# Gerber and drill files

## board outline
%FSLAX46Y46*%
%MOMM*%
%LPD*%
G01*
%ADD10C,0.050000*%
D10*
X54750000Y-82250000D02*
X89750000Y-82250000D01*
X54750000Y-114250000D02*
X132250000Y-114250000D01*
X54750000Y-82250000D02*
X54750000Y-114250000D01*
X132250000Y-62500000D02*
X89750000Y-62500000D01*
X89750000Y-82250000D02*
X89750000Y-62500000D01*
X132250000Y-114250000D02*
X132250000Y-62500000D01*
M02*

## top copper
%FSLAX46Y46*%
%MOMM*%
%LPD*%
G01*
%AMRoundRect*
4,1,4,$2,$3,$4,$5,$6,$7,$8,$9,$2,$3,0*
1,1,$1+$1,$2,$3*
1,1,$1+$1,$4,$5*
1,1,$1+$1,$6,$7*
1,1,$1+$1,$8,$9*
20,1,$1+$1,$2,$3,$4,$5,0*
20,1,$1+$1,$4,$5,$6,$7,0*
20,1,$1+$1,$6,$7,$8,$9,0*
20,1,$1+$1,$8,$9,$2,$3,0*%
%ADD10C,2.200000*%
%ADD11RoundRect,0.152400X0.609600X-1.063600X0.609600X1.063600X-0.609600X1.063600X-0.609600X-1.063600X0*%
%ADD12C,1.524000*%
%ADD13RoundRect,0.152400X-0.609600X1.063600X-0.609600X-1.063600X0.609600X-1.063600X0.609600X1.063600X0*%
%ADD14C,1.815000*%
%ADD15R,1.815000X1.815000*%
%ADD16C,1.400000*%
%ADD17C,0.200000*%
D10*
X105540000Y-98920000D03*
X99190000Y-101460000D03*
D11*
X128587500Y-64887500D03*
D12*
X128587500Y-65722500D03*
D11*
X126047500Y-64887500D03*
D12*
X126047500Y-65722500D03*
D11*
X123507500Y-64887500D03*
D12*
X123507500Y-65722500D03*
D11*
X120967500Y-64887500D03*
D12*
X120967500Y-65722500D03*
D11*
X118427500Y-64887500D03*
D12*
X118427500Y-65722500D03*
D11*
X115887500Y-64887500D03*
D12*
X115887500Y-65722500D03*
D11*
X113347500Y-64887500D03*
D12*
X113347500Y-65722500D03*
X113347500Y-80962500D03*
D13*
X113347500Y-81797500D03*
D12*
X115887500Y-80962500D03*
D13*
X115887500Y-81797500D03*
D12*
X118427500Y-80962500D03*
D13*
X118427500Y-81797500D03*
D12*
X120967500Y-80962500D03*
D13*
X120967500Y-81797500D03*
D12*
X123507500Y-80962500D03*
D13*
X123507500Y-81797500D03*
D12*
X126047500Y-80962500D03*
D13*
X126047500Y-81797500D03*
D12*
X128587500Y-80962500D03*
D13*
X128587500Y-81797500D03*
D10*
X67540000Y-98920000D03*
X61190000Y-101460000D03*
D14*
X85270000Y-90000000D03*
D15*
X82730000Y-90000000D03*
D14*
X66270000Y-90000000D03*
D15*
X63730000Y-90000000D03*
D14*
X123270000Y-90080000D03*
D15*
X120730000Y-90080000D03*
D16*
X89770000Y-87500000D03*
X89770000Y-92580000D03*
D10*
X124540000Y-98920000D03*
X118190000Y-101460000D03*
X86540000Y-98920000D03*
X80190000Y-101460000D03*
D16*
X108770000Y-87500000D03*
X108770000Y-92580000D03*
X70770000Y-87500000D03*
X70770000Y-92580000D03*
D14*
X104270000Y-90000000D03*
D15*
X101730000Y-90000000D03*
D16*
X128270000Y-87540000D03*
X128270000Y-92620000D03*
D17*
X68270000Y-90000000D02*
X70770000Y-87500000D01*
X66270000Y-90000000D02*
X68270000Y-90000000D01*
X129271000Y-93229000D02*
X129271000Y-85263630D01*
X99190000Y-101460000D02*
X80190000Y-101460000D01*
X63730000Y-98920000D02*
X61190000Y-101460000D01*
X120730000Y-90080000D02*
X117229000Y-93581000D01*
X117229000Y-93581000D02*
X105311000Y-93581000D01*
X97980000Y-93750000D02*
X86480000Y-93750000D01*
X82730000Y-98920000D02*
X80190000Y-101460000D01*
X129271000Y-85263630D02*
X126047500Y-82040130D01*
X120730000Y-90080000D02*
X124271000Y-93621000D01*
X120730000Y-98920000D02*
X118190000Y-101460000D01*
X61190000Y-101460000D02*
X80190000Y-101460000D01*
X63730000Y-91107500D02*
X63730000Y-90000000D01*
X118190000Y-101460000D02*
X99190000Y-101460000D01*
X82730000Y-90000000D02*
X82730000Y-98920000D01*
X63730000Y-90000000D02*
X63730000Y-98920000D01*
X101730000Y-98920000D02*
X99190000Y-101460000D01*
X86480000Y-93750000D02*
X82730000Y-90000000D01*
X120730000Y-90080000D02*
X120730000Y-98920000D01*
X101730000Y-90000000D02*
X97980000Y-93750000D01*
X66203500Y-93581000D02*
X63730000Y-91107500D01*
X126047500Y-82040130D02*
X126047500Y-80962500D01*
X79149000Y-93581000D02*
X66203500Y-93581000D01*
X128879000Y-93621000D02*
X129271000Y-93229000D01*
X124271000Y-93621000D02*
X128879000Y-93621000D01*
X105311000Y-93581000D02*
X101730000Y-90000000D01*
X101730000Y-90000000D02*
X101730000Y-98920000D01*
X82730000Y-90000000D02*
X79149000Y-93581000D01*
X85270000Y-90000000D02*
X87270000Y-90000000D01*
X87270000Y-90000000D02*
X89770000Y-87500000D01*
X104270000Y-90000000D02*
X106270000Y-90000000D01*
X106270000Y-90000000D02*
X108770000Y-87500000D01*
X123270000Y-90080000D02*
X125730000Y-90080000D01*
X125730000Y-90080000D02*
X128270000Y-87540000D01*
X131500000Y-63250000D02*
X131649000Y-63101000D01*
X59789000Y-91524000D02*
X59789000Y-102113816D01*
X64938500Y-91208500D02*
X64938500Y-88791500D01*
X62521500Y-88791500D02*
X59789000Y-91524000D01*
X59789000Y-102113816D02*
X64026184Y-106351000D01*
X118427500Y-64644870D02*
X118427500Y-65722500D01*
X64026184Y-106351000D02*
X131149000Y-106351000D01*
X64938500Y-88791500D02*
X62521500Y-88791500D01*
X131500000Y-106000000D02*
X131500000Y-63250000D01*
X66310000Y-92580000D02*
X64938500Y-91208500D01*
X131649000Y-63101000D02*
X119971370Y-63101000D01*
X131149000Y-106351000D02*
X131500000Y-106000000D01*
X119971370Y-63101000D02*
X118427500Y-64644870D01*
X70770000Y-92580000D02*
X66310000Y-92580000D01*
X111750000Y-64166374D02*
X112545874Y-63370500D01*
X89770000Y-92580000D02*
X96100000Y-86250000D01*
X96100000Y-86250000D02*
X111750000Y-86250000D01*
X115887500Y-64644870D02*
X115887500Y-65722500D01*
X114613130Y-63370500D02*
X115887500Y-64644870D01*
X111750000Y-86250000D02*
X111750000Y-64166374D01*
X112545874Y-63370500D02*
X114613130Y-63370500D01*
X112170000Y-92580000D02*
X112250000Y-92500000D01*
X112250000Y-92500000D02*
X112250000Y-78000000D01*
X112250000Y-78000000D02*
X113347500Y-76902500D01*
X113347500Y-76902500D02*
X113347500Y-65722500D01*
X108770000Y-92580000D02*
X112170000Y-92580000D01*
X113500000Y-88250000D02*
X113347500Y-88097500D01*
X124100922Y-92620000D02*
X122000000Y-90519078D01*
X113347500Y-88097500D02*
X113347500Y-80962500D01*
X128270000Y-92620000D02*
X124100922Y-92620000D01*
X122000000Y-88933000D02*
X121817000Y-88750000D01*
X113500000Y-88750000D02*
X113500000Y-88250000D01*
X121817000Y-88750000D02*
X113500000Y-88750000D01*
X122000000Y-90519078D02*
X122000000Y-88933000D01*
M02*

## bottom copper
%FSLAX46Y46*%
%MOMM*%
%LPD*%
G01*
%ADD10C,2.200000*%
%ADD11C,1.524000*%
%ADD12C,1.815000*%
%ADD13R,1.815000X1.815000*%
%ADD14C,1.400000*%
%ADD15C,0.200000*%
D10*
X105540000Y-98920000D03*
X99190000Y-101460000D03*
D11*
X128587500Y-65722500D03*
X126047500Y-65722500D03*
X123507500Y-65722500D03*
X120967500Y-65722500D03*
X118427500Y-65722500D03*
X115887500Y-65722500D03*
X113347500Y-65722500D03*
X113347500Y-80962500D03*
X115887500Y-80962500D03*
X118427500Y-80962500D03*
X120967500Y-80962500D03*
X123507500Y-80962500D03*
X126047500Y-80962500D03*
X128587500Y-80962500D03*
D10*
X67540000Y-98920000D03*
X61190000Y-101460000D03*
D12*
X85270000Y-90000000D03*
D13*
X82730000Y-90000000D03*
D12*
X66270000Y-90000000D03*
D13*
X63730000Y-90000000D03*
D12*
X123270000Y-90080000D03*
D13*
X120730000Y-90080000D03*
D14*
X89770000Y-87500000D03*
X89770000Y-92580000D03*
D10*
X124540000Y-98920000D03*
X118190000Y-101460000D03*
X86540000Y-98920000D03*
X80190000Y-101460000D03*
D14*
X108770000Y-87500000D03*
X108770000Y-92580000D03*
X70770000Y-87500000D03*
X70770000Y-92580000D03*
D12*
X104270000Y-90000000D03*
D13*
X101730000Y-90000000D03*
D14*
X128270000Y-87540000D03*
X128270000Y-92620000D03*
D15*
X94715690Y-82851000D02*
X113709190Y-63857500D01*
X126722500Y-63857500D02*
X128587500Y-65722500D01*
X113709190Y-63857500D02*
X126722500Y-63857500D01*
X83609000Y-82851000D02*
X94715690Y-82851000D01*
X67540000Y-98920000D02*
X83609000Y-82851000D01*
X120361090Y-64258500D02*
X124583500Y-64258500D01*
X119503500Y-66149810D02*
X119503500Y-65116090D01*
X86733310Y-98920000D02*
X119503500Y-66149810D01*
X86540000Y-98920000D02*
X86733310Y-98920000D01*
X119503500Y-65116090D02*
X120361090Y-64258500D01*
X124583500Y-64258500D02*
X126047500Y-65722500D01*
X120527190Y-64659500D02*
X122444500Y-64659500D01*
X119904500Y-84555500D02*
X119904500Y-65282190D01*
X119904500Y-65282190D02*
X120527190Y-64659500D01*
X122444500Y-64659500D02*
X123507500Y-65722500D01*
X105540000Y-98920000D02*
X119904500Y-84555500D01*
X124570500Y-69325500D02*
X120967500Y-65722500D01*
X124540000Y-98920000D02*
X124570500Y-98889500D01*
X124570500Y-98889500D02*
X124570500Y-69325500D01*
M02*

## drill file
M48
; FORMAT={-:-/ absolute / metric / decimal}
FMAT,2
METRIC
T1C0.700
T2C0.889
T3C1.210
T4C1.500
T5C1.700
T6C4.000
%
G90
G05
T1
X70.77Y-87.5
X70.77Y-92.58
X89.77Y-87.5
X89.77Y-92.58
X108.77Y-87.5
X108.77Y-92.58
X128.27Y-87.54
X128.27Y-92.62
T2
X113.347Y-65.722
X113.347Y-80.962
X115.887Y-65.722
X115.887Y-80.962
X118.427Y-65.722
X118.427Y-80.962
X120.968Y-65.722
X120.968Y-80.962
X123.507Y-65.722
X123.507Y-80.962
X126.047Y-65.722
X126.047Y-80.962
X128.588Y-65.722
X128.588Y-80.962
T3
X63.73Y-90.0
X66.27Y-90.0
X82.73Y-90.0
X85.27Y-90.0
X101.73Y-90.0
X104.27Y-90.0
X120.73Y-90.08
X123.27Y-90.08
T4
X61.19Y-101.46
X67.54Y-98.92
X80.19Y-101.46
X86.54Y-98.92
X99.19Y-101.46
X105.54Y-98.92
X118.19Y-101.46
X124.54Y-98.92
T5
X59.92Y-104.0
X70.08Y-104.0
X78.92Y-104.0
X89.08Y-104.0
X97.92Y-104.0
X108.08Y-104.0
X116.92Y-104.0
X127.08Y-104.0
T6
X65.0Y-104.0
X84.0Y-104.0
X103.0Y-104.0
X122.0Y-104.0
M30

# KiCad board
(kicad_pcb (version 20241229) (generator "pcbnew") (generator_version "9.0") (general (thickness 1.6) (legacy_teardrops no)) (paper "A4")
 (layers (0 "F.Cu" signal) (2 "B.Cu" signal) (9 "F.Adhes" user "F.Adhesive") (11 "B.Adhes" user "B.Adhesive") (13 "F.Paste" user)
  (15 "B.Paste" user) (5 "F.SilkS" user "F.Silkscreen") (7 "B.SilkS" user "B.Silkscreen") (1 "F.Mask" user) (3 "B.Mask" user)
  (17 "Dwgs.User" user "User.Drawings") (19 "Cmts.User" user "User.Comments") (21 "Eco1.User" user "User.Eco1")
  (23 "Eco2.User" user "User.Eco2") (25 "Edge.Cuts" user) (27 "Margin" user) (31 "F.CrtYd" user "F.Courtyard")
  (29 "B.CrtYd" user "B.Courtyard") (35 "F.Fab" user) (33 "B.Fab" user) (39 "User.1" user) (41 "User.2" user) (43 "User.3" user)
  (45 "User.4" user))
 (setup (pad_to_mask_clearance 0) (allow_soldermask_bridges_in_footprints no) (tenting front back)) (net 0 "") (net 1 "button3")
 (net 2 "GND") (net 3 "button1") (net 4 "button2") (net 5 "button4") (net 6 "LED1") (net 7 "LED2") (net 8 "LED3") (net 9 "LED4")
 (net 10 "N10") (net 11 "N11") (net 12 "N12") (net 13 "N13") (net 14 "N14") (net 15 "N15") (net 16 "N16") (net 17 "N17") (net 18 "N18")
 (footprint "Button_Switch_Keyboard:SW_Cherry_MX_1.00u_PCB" (layer "F.Cu") (at 105.54 98.92)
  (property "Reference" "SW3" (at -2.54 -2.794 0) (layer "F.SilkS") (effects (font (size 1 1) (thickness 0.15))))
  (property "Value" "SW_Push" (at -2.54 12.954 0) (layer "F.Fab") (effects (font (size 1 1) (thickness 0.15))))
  (pad "" np_thru_hole circle (at -7.62 5.08) (size 1.7 1.7) (drill 1.7) (layers "*.Cu" "*.Mask"))
  (pad "" np_thru_hole circle (at -2.54 5.08) (size 4 4) (drill 4) (layers "*.Cu" "*.Mask"))
  (pad "" np_thru_hole circle (at 2.54 5.08) (size 1.7 1.7) (drill 1.7) (layers "*.Cu" "*.Mask"))
  (pad "1" thru_hole circle (at 0 0) (size 2.2 2.2) (drill 1.5) (layers "*.Cu" "*.Mask") (remove_unused_layers no) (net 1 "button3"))
  (pad "2" thru_hole circle (at -6.35 2.54) (size 2.2 2.2) (drill 1.5) (layers "*.Cu" "*.Mask") (remove_unused_layers no) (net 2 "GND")))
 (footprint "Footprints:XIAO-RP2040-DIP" (layer "F.Cu") (at 120.9675 73.3425 -90)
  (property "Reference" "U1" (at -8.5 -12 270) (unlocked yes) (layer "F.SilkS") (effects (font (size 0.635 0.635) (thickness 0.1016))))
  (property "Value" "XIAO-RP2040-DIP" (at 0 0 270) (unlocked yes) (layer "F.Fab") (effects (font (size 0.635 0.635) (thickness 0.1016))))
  (pad "1" smd roundrect (at -8.455 -7.62 90) (size 2.432 1.524) (layers "F.Cu" "F.Mask") (roundrect_rratio 0.1) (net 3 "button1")
   (thermal_bridge_angle 45))
  (pad "1" thru_hole circle (at -7.62 -7.62 90) (size 1.524 1.524) (drill 0.889) (layers "*.Cu" "*.Mask") (remove_unused_layers no)
   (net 3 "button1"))
  (pad "2" smd roundrect (at -8.455 -5.08 90) (size 2.432 1.524) (layers "F.Cu" "F.Mask") (roundrect_rratio 0.1) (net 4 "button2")
   (thermal_bridge_angle 45))
  (pad "2" thru_hole circle (at -7.62 -5.08 90) (size 1.524 1.524) (drill 0.889) (layers "*.Cu" "*.Mask") (remove_unused_layers no)
   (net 4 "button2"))
  (pad "3" smd roundrect (at -8.455 -2.54 90) (size 2.432 1.524) (layers "F.Cu" "F.Mask") (roundrect_rratio 0.1) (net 1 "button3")
   (thermal_bridge_angle 45))
  (pad "3" thru_hole circle (at -7.62 -2.54 90) (size 1.524 1.524) (drill 0.889) (layers "*.Cu" "*.Mask") (remove_unused_layers no)
   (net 1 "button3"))
  (pad "4" smd roundrect (at -8.455 0 90) (size 2.432 1.524) (layers "F.Cu" "F.Mask") (roundrect_rratio 0.1) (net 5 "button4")
   (thermal_bridge_angle 45))
  (pad "4" thru_hole circle (at -7.62 0 90) (size 1.524 1.524) (drill 0.889) (layers "*.Cu" "*.Mask") (remove_unused_layers no)
   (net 5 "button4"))
  (pad "5" smd roundrect (at -8.455 2.54 90) (size 2.432 1.524) (layers "F.Cu" "F.Mask") (roundrect_rratio 0.1) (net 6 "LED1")
   (thermal_bridge_angle 45))
  (pad "5" thru_hole circle (at -7.62 2.54 90) (size 1.524 1.524) (drill 0.889) (layers "*.Cu" "*.Mask") (remove_unused_layers no)
   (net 6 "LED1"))
  (pad "6" smd roundrect (at -8.455 5.08 90) (size 2.432 1.524) (layers "F.Cu" "F.Mask") (roundrect_rratio 0.1) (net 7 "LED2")
   (thermal_bridge_angle 45))
  (pad "6" thru_hole circle (at -7.62 5.08 90) (size 1.524 1.524) (drill 0.889) (layers "*.Cu" "*.Mask") (remove_unused_layers no)
   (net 7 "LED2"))
  (pad "7" smd roundrect (at -8.455 7.62 90) (size 2.432 1.524) (layers "F.Cu" "F.Mask") (roundrect_rratio 0.1) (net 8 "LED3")
   (thermal_bridge_angle 45))
  (pad "7" thru_hole circle (at -7.62 7.62 90) (size 1.524 1.524) (drill 0.889) (layers "*.Cu" "*.Mask") (remove_unused_layers no)
   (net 8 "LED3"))
  (pad "8" thru_hole circle (at 7.62 7.62 270) (size 1.524 1.524) (drill 0.889) (layers "*.Cu" "*.Mask") (remove_unused_layers no)
   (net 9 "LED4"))
  (pad "8" smd roundrect (at 8.455 7.62 270) (size 2.432 1.524) (layers "F.Cu" "F.Mask") (roundrect_rratio 0.1) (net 9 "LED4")
   (thermal_bridge_angle 45))
  (pad "9" thru_hole circle (at 7.62 5.08 270) (size 1.524 1.524) (drill 0.889) (layers "*.Cu" "*.Mask") (remove_unused_layers no)
   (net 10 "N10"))
  (pad "9" smd roundrect (at 8.455 5.08 270) (size 2.432 1.524) (layers "F.Cu" "F.Mask") (roundrect_rratio 0.1) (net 10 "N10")
   (thermal_bridge_angle 45))
  (pad "10" thru_hole circle (at 7.62 2.54 270) (size 1.524 1.524) (drill 0.889) (layers "*.Cu" "*.Mask") (remove_unused_layers no)
   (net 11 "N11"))
  (pad "10" smd roundrect (at 8.455 2.54 270) (size 2.432 1.524) (layers "F.Cu" "F.Mask") (roundrect_rratio 0.1) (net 11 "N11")
   (thermal_bridge_angle 45))
  (pad "11" thru_hole circle (at 7.62 0 270) (size 1.524 1.524) (drill 0.889) (layers "*.Cu" "*.Mask") (remove_unused_layers no)
   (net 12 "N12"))
  (pad "11" smd roundrect (at 8.455 0 270) (size 2.432 1.524) (layers "F.Cu" "F.Mask") (roundrect_rratio 0.1) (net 12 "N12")
   (thermal_bridge_angle 45))
  (pad "12" thru_hole circle (at 7.62 -2.54 270) (size 1.524 1.524) (drill 0.889) (layers "*.Cu" "*.Mask") (remove_unused_layers no)
   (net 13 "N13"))
  (pad "12" smd roundrect (at 8.455 -2.54 270) (size 2.432 1.524) (layers "F.Cu" "F.Mask") (roundrect_rratio 0.1) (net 13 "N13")
   (thermal_bridge_angle 45))
  (pad "13" thru_hole circle (at 7.62 -5.08 270) (size 1.524 1.524) (drill 0.889) (layers "*.Cu" "*.Mask") (remove_unused_layers no)
   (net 2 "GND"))
  (pad "13" smd roundrect (at 8.455 -5.08 270) (size 2.432 1.524) (layers "F.Cu" "F.Mask") (roundrect_rratio 0.1) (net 2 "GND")
   (thermal_bridge_angle 45))
  (pad "14" thru_hole circle (at 7.62 -7.62 270) (size 1.524 1.524) (drill 0.889) (layers "*.Cu" "*.Mask") (remove_unused_layers no)
   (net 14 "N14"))
  (pad "14" smd roundrect (at 8.455 -7.62 270) (size 2.432 1.524) (layers "F.Cu" "F.Mask") (roundrect_rratio 0.1) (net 14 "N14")
   (thermal_bridge_angle 45)))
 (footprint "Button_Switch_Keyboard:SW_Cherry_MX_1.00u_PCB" (layer "F.Cu") (at 67.54 98.92)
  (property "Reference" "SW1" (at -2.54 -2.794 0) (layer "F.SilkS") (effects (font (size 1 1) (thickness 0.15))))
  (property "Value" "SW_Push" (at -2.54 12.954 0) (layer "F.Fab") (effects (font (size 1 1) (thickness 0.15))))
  (pad "" np_thru_hole circle (at -7.62 5.08) (size 1.7 1.7) (drill 1.7) (layers "*.Cu" "*.Mask"))
  (pad "" np_thru_hole circle (at -2.54 5.08) (size 4 4) (drill 4) (layers "*.Cu" "*.Mask"))
  (pad "" np_thru_hole circle (at 2.54 5.08) (size 1.7 1.7) (drill 1.7) (layers "*.Cu" "*.Mask"))
  (pad "1" thru_hole circle (at 0 0) (size 2.2 2.2) (drill 1.5) (layers "*.Cu" "*.Mask") (remove_unused_layers no) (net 3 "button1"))
  (pad "2" thru_hole circle (at -6.35 2.54) (size 2.2 2.2) (drill 1.5) (layers "*.Cu" "*.Mask") (remove_unused_layers no) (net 2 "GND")))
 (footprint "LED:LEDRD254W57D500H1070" (layer "F.Cu") (at 84 90)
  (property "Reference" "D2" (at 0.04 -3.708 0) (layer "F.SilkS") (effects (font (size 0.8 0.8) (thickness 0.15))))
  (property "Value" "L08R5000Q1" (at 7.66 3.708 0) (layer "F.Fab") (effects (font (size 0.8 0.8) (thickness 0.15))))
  (pad "A" thru_hole circle (at 1.27 0) (size 1.815 1.815) (drill 1.21) (layers "*.Cu" "*.Mask") (remove_unused_layers no) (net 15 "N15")
   (solder_mask_margin 0.102))
  (pad "C" thru_hole rect (at -1.27 0) (size 1.815 1.815) (drill 1.21) (layers "*.Cu" "*.Mask") (remove_unused_layers no) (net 2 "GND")
   (solder_mask_margin 0.102)))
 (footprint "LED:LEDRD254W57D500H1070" (layer "F.Cu") (at 65 90)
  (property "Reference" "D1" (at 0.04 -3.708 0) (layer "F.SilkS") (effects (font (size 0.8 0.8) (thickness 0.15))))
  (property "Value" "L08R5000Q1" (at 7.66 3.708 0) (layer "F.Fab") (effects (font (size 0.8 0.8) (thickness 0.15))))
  (pad "A" thru_hole circle (at 1.27 0) (size 1.815 1.815) (drill 1.21) (layers "*.Cu" "*.Mask") (remove_unused_layers no) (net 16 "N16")
   (solder_mask_margin 0.102))
  (pad "C" thru_hole rect (at -1.27 0) (size 1.815 1.815) (drill 1.21) (layers "*.Cu" "*.Mask") (remove_unused_layers no) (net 2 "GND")
   (solder_mask_margin 0.102)))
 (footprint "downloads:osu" (layer "F.Cu") (at 100 72.5)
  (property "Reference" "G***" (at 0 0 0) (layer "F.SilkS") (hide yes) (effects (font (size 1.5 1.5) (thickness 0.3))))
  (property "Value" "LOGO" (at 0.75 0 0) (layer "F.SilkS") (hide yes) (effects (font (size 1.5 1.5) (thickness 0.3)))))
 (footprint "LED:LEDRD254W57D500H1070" (layer "F.Cu") (at 122 90.08)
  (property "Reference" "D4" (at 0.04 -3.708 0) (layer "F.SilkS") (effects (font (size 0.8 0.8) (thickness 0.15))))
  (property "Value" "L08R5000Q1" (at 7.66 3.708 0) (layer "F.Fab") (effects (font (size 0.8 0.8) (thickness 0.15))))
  (pad "A" thru_hole circle (at 1.27 0) (size 1.815 1.815) (drill 1.21) (layers "*.Cu" "*.Mask") (remove_unused_layers no) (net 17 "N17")
   (solder_mask_margin 0.102))
  (pad "C" thru_hole rect (at -1.27 0) (size 1.815 1.815) (drill 1.21) (layers "*.Cu" "*.Mask") (remove_unused_layers no) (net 2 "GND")
   (solder_mask_margin 0.102)))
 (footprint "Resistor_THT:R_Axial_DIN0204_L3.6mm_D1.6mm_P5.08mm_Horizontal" (layer "F.Cu") (at 89.77 87.5 -90)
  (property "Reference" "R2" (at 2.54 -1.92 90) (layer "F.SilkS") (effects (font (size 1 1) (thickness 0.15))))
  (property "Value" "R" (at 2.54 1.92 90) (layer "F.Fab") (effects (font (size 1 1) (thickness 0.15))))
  (pad "1" thru_hole circle (at 0 0 270) (size 1.4 1.4) (drill 0.7) (layers "*.Cu" "*.Mask") (remove_unused_layers no) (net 15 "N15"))
  (pad "2" thru_hole circle (at 5.08 0 270) (size 1.4 1.4) (drill 0.7) (layers "*.Cu" "*.Mask") (remove_unused_layers no) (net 7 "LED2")))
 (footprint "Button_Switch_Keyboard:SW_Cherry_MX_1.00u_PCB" (layer "F.Cu") (at 124.54 98.92)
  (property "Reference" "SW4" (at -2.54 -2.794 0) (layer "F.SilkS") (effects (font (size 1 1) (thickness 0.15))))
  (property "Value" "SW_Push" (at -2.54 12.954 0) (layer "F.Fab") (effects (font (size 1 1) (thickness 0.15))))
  (pad "" np_thru_hole circle (at -7.62 5.08) (size 1.7 1.7) (drill 1.7) (layers "*.Cu" "*.Mask"))
  (pad "" np_thru_hole circle (at -2.54 5.08) (size 4 4) (drill 4) (layers "*.Cu" "*.Mask"))
  (pad "" np_thru_hole circle (at 2.54 5.08) (size 1.7 1.7) (drill 1.7) (layers "*.Cu" "*.Mask"))
  (pad "1" thru_hole circle (at 0 0) (size 2.2 2.2) (drill 1.5) (layers "*.Cu" "*.Mask") (remove_unused_layers no) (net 5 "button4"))
  (pad "2" thru_hole circle (at -6.35 2.54) (size 2.2 2.2) (drill 1.5) (layers "*.Cu" "*.Mask") (remove_unused_layers no) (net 2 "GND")))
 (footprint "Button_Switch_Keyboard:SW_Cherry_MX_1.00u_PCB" (layer "F.Cu") (at 86.54 98.92)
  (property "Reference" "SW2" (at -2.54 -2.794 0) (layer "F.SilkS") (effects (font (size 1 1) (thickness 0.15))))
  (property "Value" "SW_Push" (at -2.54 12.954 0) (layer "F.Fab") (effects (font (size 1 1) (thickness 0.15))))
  (pad "" np_thru_hole circle (at -7.62 5.08) (size 1.7 1.7) (drill 1.7) (layers "*.Cu" "*.Mask"))
  (pad "" np_thru_hole circle (at -2.54 5.08) (size 4 4) (drill 4) (layers "*.Cu" "*.Mask"))
  (pad "" np_thru_hole circle (at 2.54 5.08) (size 1.7 1.7) (drill 1.7) (layers "*.Cu" "*.Mask"))
  (pad "1" thru_hole circle (at 0 0) (size 2.2 2.2) (drill 1.5) (layers "*.Cu" "*.Mask") (remove_unused_layers no) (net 4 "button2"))
  (pad "2" thru_hole circle (at -6.35 2.54) (size 2.2 2.2) (drill 1.5) (layers "*.Cu" "*.Mask") (remove_unused_layers no) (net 2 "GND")))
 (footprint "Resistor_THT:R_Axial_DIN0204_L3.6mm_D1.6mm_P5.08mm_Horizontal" (layer "F.Cu") (at 108.77 87.5 -90)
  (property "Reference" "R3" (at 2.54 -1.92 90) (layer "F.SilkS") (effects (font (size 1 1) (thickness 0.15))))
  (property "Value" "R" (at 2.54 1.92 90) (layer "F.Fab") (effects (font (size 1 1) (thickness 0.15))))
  (pad "1" thru_hole circle (at 0 0 270) (size 1.4 1.4) (drill 0.7) (layers "*.Cu" "*.Mask") (remove_unused_layers no) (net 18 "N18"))
  (pad "2" thru_hole circle (at 5.08 0 270) (size 1.4 1.4) (drill 0.7) (layers "*.Cu" "*.Mask") (remove_unused_layers no) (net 8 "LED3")))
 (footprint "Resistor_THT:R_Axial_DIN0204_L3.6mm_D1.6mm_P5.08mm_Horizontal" (layer "F.Cu") (at 70.77 87.5 -90)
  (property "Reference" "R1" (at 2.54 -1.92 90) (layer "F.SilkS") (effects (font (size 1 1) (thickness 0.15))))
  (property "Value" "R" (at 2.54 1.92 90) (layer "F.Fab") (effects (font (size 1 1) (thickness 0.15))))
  (pad "1" thru_hole circle (at 0 0 270) (size 1.4 1.4) (drill 0.7) (layers "*.Cu" "*.Mask") (remove_unused_layers no) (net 16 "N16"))
  (pad "2" thru_hole circle (at 5.08 0 270) (size 1.4 1.4) (drill 0.7) (layers "*.Cu" "*.Mask") (remove_unused_layers no) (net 6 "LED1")))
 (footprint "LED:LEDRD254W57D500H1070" (layer "F.Cu") (at 103 90)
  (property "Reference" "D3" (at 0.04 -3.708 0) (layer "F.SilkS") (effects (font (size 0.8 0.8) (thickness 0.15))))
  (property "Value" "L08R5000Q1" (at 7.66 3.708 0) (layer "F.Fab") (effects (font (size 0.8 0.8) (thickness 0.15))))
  (pad "A" thru_hole circle (at 1.27 0) (size 1.815 1.815) (drill 1.21) (layers "*.Cu" "*.Mask") (remove_unused_layers no) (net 18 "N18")
   (solder_mask_margin 0.102))
  (pad "C" thru_hole rect (at -1.27 0) (size 1.815 1.815) (drill 1.21) (layers "*.Cu" "*.Mask") (remove_unused_layers no) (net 2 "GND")
   (solder_mask_margin 0.102)))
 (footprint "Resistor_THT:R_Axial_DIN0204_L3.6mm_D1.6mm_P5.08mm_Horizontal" (layer "F.Cu") (at 128.27 87.54 -90)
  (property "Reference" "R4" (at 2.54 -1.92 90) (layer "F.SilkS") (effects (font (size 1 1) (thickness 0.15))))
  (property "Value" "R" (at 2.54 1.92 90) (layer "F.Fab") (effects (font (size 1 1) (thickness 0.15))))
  (pad "1" thru_hole circle (at 0 0 270) (size 1.4 1.4) (drill 0.7) (layers "*.Cu" "*.Mask") (remove_unused_layers no) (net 17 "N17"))
  (pad "2" thru_hole circle (at 5.08 0 270) (size 1.4 1.4) (drill 0.7) (layers "*.Cu" "*.Mask") (remove_unused_layers no) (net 9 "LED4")))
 (gr_line (start 54.75 82.25) (end 89.75 82.25) (stroke (width 0.05) (type default)) (layer "Edge.Cuts"))
 (gr_line (start 54.75 114.25) (end 132.25 114.25) (stroke (width 0.05) (type default)) (layer "Edge.Cuts"))
 (gr_line (start 54.75 82.25) (end 54.75 114.25) (stroke (width 0.05) (type default)) (layer "Edge.Cuts"))
 (gr_line (start 132.25 62.5) (end 89.75 62.5) (stroke (width 0.05) (type default)) (layer "Edge.Cuts"))
 (gr_line (start 89.75 82.25) (end 89.75 62.5) (stroke (width 0.05) (type default)) (layer "Edge.Cuts"))
 (gr_line (start 132.25 114.25) (end 132.25 62.5) (stroke (width 0.05) (type default)) (layer "Edge.Cuts"))
 (segment (start 68.27 90) (end 70.77 87.5) (width 0.2) (layer "F.Cu") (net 16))
 (segment (start 66.27 90) (end 68.27 90) (width 0.2) (layer "F.Cu") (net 16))
 (segment (start 129.271 93.229) (end 129.271 85.26363) (width 0.2) (layer "F.Cu") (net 2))
 (segment (start 99.19 101.46) (end 80.19 101.46) (width 0.2) (layer "F.Cu") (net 2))
 (segment (start 63.73 98.92) (end 61.19 101.46) (width 0.2) (layer "F.Cu") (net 2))
 (segment (start 120.73 90.08) (end 117.229 93.581) (width 0.2) (layer "F.Cu") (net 2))
 (segment (start 117.229 93.581) (end 105.311 93.581) (width 0.2) (layer "F.Cu") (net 2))
 (segment (start 97.98 93.75) (end 86.48 93.75) (width 0.2) (layer "F.Cu") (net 2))
 (segment (start 82.73 98.92) (end 80.19 101.46) (width 0.2) (layer "F.Cu") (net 2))
 (segment (start 129.271 85.26363) (end 126.0475 82.04013) (width 0.2) (layer "F.Cu") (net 2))
 (segment (start 120.73 90.08) (end 124.271 93.621) (width 0.2) (layer "F.Cu") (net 2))
 (segment (start 120.73 98.92) (end 118.19 101.46) (width 0.2) (layer "F.Cu") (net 2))
 (segment (start 61.19 101.46) (end 80.19 101.46) (width 0.2) (layer "F.Cu") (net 2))
 (segment (start 63.73 91.1075) (end 63.73 90) (width 0.2) (layer "F.Cu") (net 2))
 (segment (start 118.19 101.46) (end 99.19 101.46) (width 0.2) (layer "F.Cu") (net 2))
 (segment (start 82.73 90) (end 82.73 98.92) (width 0.2) (layer "F.Cu") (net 2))
 (segment (start 63.73 90) (end 63.73 98.92) (width 0.2) (layer "F.Cu") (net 2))
 (segment (start 101.73 98.92) (end 99.19 101.46) (width 0.2) (layer "F.Cu") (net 2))
 (segment (start 86.48 93.75) (end 82.73 90) (width 0.2) (layer "F.Cu") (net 2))
 (segment (start 120.73 90.08) (end 120.73 98.92) (width 0.2) (layer "F.Cu") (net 2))
 (segment (start 101.73 90) (end 97.98 93.75) (width 0.2) (layer "F.Cu") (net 2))
 (segment (start 66.2035 93.581) (end 63.73 91.1075) (width 0.2) (layer "F.Cu") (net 2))
 (segment (start 126.0475 82.04013) (end 126.0475 80.9625) (width 0.2) (layer "F.Cu") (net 2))
 (segment (start 79.149 93.581) (end 66.2035 93.581) (width 0.2) (layer "F.Cu") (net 2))
 (segment (start 128.879 93.621) (end 129.271 93.229) (width 0.2) (layer "F.Cu") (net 2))
 (segment (start 124.271 93.621) (end 128.879 93.621) (width 0.2) (layer "F.Cu") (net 2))
 (segment (start 105.311 93.581) (end 101.73 90) (width 0.2) (layer "F.Cu") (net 2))
 (segment (start 101.73 90) (end 101.73 98.92) (width 0.2) (layer "F.Cu") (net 2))
 (segment (start 82.73 90) (end 79.149 93.581) (width 0.2) (layer "F.Cu") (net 2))
 (segment (start 85.27 90) (end 87.27 90) (width 0.2) (layer "F.Cu") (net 15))
 (segment (start 87.27 90) (end 89.77 87.5) (width 0.2) (layer "F.Cu") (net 15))
 (segment (start 104.27 90) (end 106.27 90) (width 0.2) (layer "F.Cu") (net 18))
 (segment (start 106.27 90) (end 108.77 87.5) (width 0.2) (layer "F.Cu") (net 18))
 (segment (start 123.27 90.08) (end 125.73 90.08) (width 0.2) (layer "F.Cu") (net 17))
 (segment (start 125.73 90.08) (end 128.27 87.54) (width 0.2) (layer "F.Cu") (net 17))
 (segment (start 131.5 63.25) (end 131.649 63.101) (width 0.2) (layer "F.Cu") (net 6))
 (segment (start 59.789 91.524) (end 59.789 102.113816) (width 0.2) (layer "F.Cu") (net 6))
 (segment (start 64.9385 91.2085) (end 64.9385 88.7915) (width 0.2) (layer "F.Cu") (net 6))
 (segment (start 62.5215 88.7915) (end 59.789 91.524) (width 0.2) (layer "F.Cu") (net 6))
 (segment (start 59.789 102.113816) (end 64.026184 106.351) (width 0.2) (layer "F.Cu") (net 6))
 (segment (start 118.4275 64.64487) (end 118.4275 65.7225) (width 0.2) (layer "F.Cu") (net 6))
 (segment (start 64.026184 106.351) (end 131.149 106.351) (width 0.2) (layer "F.Cu") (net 6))
 (segment (start 64.9385 88.7915) (end 62.5215 88.7915) (width 0.2) (layer "F.Cu") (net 6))
 (segment (start 131.5 106) (end 131.5 63.25) (width 0.2) (layer "F.Cu") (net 6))
 (segment (start 66.31 92.58) (end 64.9385 91.2085) (width 0.2) (layer "F.Cu") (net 6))
 (segment (start 131.649 63.101) (end 119.97137 63.101) (width 0.2) (layer "F.Cu") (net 6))
 (segment (start 131.149 106.351) (end 131.5 106) (width 0.2) (layer "F.Cu") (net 6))
 (segment (start 119.97137 63.101) (end 118.4275 64.64487) (width 0.2) (layer "F.Cu") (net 6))
 (segment (start 70.77 92.58) (end 66.31 92.58) (width 0.2) (layer "F.Cu") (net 6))
 (segment (start 111.75 64.166374) (end 112.545874 63.3705) (width 0.2) (layer "F.Cu") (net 7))
 (segment (start 89.77 92.58) (end 96.1 86.25) (width 0.2) (layer "F.Cu") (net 7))
 (segment (start 96.1 86.25) (end 111.75 86.25) (width 0.2) (layer "F.Cu") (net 7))
 (segment (start 115.8875 64.64487) (end 115.8875 65.7225) (width 0.2) (layer "F.Cu") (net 7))
 (segment (start 114.61313 63.3705) (end 115.8875 64.64487) (width 0.2) (layer "F.Cu") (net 7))
 (segment (start 111.75 86.25) (end 111.75 64.166374) (width 0.2) (layer "F.Cu") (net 7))
 (segment (start 112.545874 63.3705) (end 114.61313 63.3705) (width 0.2) (layer "F.Cu") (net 7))
 (segment (start 112.17 92.58) (end 112.25 92.5) (width 0.2) (layer "F.Cu") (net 8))
 (segment (start 112.25 92.5) (end 112.25 78) (width 0.2) (layer "F.Cu") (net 8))
 (segment (start 112.25 78) (end 113.3475 76.9025) (width 0.2) (layer "F.Cu") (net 8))
 (segment (start 113.3475 76.9025) (end 113.3475 65.7225) (width 0.2) (layer "F.Cu") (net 8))
 (segment (start 108.77 92.58) (end 112.17 92.58) (width 0.2) (layer "F.Cu") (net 8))
 (segment (start 113.5 88.25) (end 113.3475 88.0975) (width 0.2) (layer "F.Cu") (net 9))
 (segment (start 124.100922 92.62) (end 122 90.519078) (width 0.2) (layer "F.Cu") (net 9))
 (segment (start 113.3475 88.0975) (end 113.3475 80.9625) (width 0.2) (layer "F.Cu") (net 9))
 (segment (start 128.27 92.62) (end 124.100922 92.62) (width 0.2) (layer "F.Cu") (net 9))
 (segment (start 122 88.933) (end 121.817 88.75) (width 0.2) (layer "F.Cu") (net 9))
 (segment (start 113.5 88.75) (end 113.5 88.25) (width 0.2) (layer "F.Cu") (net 9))
 (segment (start 121.817 88.75) (end 113.5 88.75) (width 0.2) (layer "F.Cu") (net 9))
 (segment (start 122 90.519078) (end 122 88.933) (width 0.2) (layer "F.Cu") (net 9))
 (segment (start 94.71569 82.851) (end 113.70919 63.8575) (width 0.2) (layer "B.Cu") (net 3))
 (segment (start 126.7225 63.8575) (end 128.5875 65.7225) (width 0.2) (layer "B.Cu") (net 3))
 (segment (start 113.70919 63.8575) (end 126.7225 63.8575) (width 0.2) (layer "B.Cu") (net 3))
 (segment (start 83.609 82.851) (end 94.71569 82.851) (width 0.2) (layer "B.Cu") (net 3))
 (segment (start 67.54 98.92) (end 83.609 82.851) (width 0.2) (layer "B.Cu") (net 3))
 (segment (start 120.36109 64.2585) (end 124.5835 64.2585) (width 0.2) (layer "B.Cu") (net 4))
 (segment (start 119.5035 66.14981) (end 119.5035 65.11609) (width 0.2) (layer "B.Cu") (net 4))
 (segment (start 86.73331 98.92) (end 119.5035 66.14981) (width 0.2) (layer "B.Cu") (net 4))
 (segment (start 86.54 98.92) (end 86.73331 98.92) (width 0.2) (layer "B.Cu") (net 4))
 (segment (start 119.5035 65.11609) (end 120.36109 64.2585) (width 0.2) (layer "B.Cu") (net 4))
 (segment (start 124.5835 64.2585) (end 126.0475 65.7225) (width 0.2) (layer "B.Cu") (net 4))
 (segment (start 120.52719 64.6595) (end 122.4445 64.6595) (width 0.2) (layer "B.Cu") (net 1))
 (segment (start 119.9045 84.5555) (end 119.9045 65.28219) (width 0.2) (layer "B.Cu") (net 1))
 (segment (start 119.9045 65.28219) (end 120.52719 64.6595) (width 0.2) (layer "B.Cu") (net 1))
 (segment (start 122.4445 64.6595) (end 123.5075 65.7225) (width 0.2) (layer "B.Cu") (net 1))
 (segment (start 105.54 98.92) (end 119.9045 84.5555) (width 0.2) (layer "B.Cu") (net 1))
 (segment (start 124.5705 69.3255) (end 120.9675 65.7225) (width 0.2) (layer "B.Cu") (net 5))
 (segment (start 124.54 98.92) (end 124.5705 98.8895) (width 0.2) (layer "B.Cu") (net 5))
 (segment (start 124.5705 98.8895) (end 124.5705 69.3255) (width 0.2) (layer "B.Cu") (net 5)))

